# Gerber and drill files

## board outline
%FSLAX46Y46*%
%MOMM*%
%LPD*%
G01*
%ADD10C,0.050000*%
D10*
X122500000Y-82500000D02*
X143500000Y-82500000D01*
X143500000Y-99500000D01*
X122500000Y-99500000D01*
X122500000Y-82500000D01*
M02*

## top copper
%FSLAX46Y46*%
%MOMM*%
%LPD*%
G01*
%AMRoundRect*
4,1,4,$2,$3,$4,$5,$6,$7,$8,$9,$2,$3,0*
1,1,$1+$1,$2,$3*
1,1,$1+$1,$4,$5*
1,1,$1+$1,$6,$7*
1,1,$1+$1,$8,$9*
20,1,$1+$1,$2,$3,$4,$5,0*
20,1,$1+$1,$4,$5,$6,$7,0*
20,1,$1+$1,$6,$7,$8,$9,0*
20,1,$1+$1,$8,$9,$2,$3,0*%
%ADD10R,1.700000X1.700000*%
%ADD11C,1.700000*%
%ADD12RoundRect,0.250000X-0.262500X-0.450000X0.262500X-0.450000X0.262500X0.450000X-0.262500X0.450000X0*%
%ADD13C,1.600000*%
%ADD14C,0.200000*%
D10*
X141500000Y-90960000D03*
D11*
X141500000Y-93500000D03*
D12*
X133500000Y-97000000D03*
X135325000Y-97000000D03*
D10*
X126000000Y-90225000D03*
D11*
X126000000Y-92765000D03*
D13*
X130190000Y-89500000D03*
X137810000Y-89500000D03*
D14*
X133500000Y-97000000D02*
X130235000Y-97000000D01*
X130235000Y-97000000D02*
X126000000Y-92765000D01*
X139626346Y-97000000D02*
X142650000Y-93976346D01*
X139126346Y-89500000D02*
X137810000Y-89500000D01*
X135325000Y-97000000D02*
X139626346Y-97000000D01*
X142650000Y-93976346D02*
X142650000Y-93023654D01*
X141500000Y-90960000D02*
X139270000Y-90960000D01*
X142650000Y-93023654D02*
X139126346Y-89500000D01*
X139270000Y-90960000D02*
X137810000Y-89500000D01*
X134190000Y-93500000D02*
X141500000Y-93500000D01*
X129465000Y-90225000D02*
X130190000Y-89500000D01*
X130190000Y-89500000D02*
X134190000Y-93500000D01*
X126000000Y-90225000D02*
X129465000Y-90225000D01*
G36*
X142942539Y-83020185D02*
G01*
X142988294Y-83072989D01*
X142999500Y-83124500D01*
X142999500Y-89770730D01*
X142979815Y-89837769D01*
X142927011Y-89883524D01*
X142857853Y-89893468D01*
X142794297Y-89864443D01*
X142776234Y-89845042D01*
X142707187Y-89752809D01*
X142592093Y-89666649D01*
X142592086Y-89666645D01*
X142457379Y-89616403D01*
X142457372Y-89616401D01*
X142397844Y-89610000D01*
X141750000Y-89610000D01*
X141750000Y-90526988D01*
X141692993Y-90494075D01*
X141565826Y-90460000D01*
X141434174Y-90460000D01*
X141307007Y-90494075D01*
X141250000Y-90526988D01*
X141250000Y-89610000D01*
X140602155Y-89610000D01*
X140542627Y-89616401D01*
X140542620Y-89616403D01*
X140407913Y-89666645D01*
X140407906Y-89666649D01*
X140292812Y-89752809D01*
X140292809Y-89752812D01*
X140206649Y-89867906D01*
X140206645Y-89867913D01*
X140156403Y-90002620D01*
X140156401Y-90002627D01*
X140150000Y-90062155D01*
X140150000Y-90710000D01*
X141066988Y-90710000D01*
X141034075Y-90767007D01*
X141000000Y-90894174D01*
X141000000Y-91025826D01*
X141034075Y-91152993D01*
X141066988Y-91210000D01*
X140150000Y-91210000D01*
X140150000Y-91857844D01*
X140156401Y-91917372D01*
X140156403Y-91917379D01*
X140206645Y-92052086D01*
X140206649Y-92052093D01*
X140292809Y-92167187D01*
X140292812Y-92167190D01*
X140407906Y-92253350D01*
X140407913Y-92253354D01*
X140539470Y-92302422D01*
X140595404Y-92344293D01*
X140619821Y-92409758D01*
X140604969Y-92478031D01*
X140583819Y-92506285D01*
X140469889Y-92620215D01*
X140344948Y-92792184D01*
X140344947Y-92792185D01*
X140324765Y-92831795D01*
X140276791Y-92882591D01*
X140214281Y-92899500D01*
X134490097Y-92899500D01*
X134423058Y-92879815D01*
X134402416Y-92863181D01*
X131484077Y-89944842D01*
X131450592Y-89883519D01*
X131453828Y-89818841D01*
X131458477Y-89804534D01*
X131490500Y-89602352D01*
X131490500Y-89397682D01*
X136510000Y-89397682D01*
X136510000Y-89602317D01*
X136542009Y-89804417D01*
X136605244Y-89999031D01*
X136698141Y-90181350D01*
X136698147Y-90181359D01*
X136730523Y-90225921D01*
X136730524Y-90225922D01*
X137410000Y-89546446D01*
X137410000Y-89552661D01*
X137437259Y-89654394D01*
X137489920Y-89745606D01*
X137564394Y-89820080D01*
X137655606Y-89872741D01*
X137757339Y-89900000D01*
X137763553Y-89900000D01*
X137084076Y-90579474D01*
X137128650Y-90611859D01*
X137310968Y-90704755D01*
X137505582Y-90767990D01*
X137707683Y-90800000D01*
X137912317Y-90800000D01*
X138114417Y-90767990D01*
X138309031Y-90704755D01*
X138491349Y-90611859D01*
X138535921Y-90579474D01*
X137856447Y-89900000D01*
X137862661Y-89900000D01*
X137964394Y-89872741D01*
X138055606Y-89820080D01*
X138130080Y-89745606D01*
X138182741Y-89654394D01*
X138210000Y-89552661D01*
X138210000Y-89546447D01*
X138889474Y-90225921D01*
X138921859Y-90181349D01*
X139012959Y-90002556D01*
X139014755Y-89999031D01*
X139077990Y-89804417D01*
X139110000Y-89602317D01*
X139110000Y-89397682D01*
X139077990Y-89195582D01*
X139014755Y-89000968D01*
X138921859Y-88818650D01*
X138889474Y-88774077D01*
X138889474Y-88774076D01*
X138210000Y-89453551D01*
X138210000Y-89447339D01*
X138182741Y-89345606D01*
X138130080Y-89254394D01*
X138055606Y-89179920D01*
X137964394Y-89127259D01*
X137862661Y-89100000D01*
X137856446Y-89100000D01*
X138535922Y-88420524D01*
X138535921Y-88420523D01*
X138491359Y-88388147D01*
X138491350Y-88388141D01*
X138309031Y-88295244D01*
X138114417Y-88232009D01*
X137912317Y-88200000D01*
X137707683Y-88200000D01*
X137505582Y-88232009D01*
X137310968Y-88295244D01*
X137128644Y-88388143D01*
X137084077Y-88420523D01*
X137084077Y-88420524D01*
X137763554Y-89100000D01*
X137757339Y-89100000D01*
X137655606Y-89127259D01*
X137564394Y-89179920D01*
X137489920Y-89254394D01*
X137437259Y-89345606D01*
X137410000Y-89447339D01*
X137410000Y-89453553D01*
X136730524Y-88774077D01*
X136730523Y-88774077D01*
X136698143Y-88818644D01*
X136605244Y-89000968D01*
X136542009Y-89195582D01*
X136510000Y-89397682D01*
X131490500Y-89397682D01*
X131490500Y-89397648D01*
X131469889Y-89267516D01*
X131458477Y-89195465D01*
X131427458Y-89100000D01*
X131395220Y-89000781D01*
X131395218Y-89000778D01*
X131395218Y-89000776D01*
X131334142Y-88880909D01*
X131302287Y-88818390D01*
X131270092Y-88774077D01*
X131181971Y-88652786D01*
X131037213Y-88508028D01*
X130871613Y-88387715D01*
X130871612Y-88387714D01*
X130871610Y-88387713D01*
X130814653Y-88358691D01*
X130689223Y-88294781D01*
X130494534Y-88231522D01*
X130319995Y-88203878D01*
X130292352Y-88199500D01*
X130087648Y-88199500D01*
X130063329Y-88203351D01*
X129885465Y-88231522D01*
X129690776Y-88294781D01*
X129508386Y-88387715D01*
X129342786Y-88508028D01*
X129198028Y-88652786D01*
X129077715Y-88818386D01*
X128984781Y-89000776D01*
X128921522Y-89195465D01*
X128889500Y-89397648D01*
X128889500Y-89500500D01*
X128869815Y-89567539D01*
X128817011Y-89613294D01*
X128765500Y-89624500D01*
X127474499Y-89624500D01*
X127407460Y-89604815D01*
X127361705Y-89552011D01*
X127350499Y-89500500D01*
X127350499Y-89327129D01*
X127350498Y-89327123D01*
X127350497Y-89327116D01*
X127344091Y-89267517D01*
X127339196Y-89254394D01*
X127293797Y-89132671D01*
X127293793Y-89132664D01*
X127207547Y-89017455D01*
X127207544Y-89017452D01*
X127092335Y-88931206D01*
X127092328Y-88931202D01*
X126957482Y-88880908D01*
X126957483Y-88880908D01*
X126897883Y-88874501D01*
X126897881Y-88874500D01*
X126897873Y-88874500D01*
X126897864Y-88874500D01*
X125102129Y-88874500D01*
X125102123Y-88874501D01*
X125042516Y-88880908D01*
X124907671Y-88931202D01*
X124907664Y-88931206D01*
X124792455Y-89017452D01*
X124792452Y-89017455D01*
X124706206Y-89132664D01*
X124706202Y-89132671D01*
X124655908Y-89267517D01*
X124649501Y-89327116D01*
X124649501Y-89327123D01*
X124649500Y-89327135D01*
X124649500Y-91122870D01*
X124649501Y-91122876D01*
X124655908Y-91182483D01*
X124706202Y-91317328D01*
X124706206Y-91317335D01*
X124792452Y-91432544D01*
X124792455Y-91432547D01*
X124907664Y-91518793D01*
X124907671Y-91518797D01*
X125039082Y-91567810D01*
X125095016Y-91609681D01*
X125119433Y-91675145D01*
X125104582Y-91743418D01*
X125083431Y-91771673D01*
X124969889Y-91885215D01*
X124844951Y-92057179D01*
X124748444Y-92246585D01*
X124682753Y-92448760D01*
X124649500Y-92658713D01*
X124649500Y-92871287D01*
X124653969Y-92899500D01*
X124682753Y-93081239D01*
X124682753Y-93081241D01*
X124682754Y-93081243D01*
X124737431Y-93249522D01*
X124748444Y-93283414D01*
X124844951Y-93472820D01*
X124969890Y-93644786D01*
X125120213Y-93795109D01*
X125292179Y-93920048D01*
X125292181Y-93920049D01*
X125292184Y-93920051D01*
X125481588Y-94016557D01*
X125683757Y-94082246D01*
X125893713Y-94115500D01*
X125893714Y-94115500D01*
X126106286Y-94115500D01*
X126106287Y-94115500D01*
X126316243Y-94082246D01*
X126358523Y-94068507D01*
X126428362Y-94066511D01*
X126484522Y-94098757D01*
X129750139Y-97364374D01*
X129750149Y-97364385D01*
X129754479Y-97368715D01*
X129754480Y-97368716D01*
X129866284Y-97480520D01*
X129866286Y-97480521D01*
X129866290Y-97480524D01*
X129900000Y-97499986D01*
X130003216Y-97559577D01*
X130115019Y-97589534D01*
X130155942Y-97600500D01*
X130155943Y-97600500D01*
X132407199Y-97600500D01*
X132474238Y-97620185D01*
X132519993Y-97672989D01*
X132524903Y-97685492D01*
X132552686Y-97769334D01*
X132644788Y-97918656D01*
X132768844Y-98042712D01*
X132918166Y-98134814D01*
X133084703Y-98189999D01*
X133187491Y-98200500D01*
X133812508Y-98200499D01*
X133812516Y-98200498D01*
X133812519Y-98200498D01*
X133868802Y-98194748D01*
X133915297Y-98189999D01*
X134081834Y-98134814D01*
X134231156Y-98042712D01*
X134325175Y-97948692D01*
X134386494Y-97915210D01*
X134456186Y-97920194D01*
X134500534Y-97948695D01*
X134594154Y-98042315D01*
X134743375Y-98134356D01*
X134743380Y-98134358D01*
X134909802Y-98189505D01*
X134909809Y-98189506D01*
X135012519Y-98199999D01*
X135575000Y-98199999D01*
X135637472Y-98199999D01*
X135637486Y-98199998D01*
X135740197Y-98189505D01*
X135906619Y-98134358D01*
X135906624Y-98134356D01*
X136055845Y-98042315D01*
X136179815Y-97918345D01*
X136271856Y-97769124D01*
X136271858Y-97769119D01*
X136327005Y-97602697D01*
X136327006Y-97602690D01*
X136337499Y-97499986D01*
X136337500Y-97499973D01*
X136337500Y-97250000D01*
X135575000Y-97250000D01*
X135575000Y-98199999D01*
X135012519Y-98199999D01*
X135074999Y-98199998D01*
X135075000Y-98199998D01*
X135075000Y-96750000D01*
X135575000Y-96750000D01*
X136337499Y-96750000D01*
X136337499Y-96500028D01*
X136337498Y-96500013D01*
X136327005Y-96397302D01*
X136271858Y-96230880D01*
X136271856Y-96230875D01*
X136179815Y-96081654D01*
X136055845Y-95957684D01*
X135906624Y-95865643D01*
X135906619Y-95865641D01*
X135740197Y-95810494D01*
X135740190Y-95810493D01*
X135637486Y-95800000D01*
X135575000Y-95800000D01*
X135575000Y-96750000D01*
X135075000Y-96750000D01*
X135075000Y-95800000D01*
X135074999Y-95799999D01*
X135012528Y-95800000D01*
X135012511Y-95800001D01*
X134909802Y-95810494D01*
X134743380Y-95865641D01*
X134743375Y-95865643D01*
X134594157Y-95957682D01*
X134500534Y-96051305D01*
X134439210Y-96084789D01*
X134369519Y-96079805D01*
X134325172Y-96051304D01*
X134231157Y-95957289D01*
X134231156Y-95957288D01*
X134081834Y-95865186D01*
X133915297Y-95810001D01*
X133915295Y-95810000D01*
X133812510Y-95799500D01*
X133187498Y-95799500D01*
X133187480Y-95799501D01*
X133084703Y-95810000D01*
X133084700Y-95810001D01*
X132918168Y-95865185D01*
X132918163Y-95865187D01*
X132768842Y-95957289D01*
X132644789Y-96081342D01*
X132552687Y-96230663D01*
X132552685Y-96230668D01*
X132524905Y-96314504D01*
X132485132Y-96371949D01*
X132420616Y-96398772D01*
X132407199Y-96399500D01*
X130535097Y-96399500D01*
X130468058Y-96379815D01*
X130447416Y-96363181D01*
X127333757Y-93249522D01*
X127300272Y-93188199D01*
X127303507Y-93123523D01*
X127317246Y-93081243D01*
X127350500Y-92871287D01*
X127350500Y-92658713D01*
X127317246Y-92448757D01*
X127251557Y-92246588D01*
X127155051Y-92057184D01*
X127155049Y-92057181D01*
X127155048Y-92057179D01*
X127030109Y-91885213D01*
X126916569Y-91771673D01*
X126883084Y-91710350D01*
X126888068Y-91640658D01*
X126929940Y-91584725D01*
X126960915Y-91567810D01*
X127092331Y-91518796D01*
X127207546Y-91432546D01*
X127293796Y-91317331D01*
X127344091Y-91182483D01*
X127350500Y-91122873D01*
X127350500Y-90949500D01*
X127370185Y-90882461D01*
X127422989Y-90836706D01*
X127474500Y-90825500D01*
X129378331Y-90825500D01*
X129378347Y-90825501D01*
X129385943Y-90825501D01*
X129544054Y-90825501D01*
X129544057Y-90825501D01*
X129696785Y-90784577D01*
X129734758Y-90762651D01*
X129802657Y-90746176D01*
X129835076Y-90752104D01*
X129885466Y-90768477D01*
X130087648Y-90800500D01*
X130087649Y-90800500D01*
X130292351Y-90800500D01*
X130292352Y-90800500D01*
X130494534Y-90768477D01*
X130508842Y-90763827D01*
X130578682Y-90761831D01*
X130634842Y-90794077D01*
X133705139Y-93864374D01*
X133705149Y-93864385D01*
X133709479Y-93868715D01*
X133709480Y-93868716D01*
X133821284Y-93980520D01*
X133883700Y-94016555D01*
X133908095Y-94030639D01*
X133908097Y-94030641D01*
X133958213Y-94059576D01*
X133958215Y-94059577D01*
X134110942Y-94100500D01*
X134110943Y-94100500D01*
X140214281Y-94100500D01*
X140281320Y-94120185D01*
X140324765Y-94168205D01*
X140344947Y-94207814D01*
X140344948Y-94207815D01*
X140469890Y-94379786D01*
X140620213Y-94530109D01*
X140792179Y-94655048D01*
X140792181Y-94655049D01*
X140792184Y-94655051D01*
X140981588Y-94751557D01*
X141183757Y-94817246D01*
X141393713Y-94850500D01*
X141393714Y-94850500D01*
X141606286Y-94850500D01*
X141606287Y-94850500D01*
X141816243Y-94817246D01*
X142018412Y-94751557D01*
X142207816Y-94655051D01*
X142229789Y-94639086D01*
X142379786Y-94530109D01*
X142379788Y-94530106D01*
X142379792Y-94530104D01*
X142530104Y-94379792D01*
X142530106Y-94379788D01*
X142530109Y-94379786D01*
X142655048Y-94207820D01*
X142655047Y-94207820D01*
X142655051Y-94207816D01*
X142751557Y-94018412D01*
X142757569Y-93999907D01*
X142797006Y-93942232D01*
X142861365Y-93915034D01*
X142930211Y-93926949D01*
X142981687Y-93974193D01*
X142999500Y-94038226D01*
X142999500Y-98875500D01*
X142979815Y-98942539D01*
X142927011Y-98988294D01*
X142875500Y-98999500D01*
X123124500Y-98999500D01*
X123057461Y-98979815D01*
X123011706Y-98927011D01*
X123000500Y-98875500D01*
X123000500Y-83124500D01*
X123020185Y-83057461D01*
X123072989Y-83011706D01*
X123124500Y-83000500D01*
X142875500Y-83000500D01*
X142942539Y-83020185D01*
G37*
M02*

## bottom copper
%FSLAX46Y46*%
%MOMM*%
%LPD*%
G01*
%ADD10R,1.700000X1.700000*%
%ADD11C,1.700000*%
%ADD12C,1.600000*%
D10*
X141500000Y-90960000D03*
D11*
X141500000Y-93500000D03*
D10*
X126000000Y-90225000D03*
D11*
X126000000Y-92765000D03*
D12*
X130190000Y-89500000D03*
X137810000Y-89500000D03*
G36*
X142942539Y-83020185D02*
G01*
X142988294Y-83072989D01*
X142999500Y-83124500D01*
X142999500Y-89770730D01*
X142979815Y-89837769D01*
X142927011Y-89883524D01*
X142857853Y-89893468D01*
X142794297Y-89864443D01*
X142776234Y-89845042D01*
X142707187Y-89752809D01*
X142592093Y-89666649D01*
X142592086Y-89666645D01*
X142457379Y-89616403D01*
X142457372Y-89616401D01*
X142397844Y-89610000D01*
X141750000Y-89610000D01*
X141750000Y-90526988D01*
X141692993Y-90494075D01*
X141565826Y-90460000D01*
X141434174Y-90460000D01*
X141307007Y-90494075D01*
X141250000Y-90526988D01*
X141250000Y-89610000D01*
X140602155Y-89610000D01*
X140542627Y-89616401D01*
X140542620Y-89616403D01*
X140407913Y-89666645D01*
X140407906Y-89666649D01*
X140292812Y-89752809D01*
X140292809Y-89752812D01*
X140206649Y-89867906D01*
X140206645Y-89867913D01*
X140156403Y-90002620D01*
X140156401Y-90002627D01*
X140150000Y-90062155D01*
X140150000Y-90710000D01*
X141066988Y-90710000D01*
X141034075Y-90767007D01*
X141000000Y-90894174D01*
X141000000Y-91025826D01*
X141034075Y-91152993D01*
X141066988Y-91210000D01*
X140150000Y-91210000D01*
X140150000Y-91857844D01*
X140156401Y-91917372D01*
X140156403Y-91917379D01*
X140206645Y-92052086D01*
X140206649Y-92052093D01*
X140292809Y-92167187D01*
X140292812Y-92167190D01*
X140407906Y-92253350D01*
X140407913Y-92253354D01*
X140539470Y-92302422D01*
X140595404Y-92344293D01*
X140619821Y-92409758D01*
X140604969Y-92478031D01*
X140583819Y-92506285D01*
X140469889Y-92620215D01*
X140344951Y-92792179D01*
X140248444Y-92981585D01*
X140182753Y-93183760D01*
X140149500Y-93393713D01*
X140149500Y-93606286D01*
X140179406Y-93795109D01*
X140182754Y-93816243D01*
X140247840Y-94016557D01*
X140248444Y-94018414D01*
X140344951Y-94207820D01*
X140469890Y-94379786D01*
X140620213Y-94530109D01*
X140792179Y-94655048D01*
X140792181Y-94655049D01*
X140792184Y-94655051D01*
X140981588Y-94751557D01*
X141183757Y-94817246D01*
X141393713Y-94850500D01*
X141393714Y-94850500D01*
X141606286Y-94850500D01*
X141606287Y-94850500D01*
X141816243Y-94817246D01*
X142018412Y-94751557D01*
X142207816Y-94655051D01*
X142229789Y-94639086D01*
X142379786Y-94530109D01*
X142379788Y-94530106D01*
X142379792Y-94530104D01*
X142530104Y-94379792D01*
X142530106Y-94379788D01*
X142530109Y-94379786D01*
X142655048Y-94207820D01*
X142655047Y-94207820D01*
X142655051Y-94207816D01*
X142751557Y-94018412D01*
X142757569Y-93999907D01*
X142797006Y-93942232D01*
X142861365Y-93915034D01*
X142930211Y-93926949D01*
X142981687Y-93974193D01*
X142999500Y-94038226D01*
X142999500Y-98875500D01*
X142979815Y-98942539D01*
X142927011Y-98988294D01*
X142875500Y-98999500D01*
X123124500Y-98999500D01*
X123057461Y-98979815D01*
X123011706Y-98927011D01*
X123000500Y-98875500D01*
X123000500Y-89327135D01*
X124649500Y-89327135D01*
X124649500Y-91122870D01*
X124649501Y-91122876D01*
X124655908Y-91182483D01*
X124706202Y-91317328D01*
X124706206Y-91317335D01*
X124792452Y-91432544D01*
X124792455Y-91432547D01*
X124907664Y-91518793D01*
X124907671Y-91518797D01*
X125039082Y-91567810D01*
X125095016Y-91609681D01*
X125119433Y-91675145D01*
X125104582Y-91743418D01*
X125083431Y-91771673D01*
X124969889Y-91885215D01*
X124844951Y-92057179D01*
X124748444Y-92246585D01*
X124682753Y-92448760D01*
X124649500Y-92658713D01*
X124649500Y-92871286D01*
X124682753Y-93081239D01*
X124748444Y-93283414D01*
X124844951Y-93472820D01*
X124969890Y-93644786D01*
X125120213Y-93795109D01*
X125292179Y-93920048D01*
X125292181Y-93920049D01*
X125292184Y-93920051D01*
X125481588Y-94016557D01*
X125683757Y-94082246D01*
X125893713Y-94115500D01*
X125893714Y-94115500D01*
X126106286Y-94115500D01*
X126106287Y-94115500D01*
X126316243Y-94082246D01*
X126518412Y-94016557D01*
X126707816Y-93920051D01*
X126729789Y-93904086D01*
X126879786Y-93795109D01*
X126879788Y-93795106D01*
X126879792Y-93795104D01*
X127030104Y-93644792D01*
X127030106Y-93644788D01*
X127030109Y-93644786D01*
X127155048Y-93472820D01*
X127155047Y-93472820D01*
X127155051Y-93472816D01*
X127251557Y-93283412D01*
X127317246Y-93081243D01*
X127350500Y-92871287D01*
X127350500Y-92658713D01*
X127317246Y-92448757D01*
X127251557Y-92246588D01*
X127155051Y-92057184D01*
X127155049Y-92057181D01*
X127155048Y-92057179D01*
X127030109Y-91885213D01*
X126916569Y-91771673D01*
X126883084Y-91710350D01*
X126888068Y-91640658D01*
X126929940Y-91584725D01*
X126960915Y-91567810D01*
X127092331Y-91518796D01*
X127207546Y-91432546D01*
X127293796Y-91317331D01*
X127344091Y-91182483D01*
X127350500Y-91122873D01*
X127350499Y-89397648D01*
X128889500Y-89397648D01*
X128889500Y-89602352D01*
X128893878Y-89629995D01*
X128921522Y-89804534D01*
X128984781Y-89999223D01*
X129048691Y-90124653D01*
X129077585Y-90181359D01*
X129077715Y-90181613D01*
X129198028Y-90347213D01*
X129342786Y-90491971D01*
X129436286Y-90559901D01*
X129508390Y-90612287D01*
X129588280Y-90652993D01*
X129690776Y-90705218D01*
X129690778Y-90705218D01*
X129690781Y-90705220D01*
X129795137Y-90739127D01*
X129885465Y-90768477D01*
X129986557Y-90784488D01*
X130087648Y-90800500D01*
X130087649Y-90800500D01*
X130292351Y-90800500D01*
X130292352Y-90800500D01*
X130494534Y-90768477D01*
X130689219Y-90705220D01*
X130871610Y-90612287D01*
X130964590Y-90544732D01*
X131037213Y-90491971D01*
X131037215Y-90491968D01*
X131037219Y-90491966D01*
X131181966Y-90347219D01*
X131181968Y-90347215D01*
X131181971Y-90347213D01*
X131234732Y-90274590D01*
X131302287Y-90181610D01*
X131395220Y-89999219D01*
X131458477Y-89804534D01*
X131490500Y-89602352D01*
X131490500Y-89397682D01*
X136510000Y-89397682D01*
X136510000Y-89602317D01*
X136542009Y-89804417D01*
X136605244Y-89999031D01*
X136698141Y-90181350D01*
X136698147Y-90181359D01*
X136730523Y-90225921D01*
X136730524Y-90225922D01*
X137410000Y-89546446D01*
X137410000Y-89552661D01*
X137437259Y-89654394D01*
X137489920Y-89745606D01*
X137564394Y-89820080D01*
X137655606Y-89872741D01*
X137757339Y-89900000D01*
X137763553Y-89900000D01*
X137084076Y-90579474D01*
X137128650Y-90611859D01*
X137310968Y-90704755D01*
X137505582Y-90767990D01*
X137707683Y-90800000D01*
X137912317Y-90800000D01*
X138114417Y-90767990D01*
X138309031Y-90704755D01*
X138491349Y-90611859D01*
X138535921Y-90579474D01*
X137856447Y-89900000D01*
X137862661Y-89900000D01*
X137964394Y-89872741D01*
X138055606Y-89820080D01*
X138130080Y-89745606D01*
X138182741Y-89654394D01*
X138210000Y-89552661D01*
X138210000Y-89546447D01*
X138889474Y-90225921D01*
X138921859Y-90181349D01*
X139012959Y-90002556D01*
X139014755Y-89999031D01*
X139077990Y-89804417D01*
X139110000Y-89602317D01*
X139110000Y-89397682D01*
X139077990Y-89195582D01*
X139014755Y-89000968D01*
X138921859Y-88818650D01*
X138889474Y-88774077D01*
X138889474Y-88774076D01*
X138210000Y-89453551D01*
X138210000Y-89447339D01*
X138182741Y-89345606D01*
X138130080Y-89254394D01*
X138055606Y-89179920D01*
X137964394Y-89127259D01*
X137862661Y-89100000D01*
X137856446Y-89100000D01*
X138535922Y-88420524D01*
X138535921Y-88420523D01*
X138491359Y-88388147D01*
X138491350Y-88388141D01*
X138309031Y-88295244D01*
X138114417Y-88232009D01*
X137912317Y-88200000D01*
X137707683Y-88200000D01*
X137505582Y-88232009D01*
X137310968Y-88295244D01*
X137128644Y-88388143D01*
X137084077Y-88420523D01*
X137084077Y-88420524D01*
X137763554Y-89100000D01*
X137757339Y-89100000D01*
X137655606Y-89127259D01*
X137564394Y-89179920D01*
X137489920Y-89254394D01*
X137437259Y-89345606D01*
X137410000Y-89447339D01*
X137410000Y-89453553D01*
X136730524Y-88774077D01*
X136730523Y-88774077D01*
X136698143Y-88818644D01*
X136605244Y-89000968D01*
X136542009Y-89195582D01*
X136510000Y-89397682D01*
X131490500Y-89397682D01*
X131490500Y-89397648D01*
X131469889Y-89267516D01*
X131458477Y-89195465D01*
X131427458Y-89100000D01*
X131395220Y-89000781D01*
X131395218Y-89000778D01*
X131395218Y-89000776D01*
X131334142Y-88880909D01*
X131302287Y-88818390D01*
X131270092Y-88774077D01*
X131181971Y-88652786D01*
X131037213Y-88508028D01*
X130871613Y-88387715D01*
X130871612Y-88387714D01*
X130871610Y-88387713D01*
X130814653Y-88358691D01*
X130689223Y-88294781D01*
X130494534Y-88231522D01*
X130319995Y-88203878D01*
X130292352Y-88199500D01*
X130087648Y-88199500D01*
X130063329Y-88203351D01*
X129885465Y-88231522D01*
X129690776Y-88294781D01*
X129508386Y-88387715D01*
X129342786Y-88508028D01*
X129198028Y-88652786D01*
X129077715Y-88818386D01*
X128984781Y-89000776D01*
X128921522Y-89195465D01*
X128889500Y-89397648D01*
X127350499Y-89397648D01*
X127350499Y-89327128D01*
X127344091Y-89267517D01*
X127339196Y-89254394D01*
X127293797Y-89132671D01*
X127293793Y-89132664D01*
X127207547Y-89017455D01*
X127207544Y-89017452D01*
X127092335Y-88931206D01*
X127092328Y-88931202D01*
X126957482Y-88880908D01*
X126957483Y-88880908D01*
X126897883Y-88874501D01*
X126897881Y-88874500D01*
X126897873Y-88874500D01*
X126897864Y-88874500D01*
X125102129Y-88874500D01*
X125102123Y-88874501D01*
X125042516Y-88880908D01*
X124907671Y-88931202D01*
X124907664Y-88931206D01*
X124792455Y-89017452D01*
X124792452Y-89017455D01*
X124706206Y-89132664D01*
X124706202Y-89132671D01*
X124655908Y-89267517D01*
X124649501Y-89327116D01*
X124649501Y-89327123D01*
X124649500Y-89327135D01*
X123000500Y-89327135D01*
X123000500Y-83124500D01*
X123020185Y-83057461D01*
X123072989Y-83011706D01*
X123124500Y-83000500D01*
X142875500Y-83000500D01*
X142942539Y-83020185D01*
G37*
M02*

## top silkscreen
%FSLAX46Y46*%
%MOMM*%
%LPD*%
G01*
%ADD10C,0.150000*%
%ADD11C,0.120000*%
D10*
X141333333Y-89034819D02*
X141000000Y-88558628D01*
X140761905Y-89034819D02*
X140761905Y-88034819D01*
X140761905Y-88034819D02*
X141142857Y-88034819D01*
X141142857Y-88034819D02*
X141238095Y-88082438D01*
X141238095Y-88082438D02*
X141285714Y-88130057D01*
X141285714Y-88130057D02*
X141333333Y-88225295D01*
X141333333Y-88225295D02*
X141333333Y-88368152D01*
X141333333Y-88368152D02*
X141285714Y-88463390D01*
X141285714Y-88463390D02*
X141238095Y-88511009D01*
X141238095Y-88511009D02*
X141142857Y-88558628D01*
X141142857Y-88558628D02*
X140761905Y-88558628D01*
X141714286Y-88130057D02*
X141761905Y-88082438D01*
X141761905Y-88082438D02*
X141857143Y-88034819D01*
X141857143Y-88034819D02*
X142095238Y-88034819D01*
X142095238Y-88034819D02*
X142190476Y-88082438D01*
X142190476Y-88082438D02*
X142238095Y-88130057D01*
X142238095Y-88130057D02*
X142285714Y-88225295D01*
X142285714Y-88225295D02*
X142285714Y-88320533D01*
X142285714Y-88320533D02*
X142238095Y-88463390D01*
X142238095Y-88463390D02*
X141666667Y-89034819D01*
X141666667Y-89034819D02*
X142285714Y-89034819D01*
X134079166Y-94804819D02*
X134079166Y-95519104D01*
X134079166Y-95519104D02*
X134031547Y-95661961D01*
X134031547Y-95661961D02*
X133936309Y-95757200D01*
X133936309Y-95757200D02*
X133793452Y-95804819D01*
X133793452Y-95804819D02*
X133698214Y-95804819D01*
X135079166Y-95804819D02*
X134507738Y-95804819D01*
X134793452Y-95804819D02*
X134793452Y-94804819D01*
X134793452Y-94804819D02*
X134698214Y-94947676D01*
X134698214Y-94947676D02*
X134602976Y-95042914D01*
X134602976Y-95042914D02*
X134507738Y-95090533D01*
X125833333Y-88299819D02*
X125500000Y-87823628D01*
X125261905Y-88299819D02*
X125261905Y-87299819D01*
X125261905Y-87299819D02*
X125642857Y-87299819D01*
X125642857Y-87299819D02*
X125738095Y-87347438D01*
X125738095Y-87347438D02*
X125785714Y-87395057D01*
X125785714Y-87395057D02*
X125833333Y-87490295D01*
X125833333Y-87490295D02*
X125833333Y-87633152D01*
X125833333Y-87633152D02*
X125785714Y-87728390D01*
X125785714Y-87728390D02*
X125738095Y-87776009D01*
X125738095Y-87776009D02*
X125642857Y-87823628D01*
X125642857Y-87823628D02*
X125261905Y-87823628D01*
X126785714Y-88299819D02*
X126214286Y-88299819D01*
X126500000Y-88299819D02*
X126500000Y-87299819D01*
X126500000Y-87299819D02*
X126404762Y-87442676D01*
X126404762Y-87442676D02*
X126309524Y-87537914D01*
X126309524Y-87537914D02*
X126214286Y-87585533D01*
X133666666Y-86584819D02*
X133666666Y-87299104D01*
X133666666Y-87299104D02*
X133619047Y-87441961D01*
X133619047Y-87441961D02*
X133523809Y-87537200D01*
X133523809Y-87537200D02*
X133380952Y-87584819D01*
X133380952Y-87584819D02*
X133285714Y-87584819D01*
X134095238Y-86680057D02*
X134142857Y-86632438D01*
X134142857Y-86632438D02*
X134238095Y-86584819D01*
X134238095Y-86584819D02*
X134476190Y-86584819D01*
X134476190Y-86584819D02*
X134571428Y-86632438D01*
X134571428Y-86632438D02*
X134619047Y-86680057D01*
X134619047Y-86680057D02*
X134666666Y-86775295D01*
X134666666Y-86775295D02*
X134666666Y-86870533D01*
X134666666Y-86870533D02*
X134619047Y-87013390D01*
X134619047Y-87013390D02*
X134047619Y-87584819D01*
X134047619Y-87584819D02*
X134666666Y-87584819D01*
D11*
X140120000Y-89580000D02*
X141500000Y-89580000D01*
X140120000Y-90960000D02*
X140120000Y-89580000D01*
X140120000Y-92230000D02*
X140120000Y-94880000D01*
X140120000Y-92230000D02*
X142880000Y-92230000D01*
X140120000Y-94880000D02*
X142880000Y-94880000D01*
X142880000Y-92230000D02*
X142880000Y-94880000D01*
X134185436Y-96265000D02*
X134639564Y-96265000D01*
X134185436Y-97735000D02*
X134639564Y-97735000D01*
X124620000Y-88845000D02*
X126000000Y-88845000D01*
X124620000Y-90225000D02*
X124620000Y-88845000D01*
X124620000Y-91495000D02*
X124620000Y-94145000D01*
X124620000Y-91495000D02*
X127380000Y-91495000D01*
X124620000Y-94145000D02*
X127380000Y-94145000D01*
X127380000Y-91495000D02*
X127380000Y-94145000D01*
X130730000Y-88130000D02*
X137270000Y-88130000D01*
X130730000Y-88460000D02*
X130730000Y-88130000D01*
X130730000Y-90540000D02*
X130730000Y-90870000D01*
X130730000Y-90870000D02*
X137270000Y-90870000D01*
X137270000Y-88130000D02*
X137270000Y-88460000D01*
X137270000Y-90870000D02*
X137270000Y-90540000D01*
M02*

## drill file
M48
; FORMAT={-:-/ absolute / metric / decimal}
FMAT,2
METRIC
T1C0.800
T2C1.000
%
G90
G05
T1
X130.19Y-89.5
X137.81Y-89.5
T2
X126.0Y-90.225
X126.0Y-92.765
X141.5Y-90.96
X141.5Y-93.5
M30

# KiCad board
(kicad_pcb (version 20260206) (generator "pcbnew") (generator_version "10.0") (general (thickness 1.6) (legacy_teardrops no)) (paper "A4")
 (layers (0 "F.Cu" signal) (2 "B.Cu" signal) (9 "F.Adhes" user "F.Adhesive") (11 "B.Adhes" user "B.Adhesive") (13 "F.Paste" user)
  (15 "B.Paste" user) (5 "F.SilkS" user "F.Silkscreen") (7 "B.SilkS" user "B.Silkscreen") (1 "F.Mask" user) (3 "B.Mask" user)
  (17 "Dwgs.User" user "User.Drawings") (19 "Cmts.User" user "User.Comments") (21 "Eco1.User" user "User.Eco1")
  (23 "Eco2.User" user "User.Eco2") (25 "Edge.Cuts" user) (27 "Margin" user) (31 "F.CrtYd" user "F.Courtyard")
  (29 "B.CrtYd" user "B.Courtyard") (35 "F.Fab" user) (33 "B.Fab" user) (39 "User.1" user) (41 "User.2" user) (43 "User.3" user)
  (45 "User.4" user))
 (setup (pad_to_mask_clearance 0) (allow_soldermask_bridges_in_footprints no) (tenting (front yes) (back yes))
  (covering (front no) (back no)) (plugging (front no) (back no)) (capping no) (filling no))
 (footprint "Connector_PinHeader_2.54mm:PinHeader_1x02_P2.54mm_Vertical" (layer "F.Cu") (at 141.5 90.96)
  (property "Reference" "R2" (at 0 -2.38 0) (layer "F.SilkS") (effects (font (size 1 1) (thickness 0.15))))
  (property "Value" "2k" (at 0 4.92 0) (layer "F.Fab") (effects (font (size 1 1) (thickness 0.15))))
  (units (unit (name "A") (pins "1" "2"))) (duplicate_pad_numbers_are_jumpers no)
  (fp_line (start -1.38 -1.38) (end 0 -1.38) (stroke (width 0.12) (type solid)) (layer "F.SilkS"))
  (fp_line (start -1.38 0) (end -1.38 -1.38) (stroke (width 0.12) (type solid)) (layer "F.SilkS"))
  (fp_line (start -1.38 1.27) (end -1.38 3.92) (stroke (width 0.12) (type solid)) (layer "F.SilkS"))
  (fp_line (start -1.38 1.27) (end 1.38 1.27) (stroke (width 0.12) (type solid)) (layer "F.SilkS"))
  (fp_line (start -1.38 3.92) (end 1.38 3.92) (stroke (width 0.12) (type solid)) (layer "F.SilkS"))
  (fp_line (start 1.38 1.27) (end 1.38 3.92) (stroke (width 0.12) (type solid)) (layer "F.SilkS"))
  (pad "1" thru_hole rect (at 0 0) (size 1.7 1.7) (drill 1) (layers "*.Cu" "*.Mask") (remove_unused_layers no) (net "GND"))
  (pad "2" thru_hole circle (at 0 2.54) (size 1.7 1.7) (drill 1) (layers "*.Cu" "*.Mask") (remove_unused_layers no) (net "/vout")))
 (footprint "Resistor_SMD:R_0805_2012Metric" (layer "F.Cu") (at 134.4125 97)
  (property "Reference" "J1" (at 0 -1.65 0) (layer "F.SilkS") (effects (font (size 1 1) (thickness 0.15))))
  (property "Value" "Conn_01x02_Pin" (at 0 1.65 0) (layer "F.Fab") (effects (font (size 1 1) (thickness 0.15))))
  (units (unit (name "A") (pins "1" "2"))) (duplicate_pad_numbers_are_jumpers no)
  (fp_line (start -0.227064 -0.735) (end 0.227064 -0.735) (stroke (width 0.12) (type solid)) (layer "F.SilkS"))
  (fp_line (start -0.227064 0.735) (end 0.227064 0.735) (stroke (width 0.12) (type solid)) (layer "F.SilkS"))
  (pad "1" smd roundrect (at -0.9125 0) (size 1.025 1.4) (layers "F.Cu" "F.Mask" "F.Paste") (roundrect_rratio 0.243902)
   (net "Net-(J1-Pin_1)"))
  (pad "2" smd roundrect (at 0.9125 0) (size 1.025 1.4) (layers "F.Cu" "F.Mask" "F.Paste") (roundrect_rratio 0.243902) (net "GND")))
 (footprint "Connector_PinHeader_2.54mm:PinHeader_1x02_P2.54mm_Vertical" (layer "F.Cu") (at 126 90.225)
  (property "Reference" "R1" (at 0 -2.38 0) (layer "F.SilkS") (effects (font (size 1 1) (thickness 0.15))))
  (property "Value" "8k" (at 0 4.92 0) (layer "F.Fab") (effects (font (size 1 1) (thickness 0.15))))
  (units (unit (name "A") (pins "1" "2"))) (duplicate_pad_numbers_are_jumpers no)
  (fp_line (start -1.38 -1.38) (end 0 -1.38) (stroke (width 0.12) (type solid)) (layer "F.SilkS"))
  (fp_line (start -1.38 0) (end -1.38 -1.38) (stroke (width 0.12) (type solid)) (layer "F.SilkS"))
  (fp_line (start -1.38 1.27) (end -1.38 3.92) (stroke (width 0.12) (type solid)) (layer "F.SilkS"))
  (fp_line (start -1.38 1.27) (end 1.38 1.27) (stroke (width 0.12) (type solid)) (layer "F.SilkS"))
  (fp_line (start -1.38 3.92) (end 1.38 3.92) (stroke (width 0.12) (type solid)) (layer "F.SilkS"))
  (fp_line (start 1.38 1.27) (end 1.38 3.92) (stroke (width 0.12) (type solid)) (layer "F.SilkS"))
  (pad "1" thru_hole rect (at 0 0) (size 1.7 1.7) (drill 1) (layers "*.Cu" "*.Mask") (remove_unused_layers no) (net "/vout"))
  (pad "2" thru_hole circle (at 0 2.54) (size 1.7 1.7) (drill 1) (layers "*.Cu" "*.Mask") (remove_unused_layers no) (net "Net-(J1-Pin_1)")))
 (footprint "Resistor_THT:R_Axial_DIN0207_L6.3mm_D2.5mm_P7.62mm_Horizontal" (layer "F.Cu") (at 130.19 89.5)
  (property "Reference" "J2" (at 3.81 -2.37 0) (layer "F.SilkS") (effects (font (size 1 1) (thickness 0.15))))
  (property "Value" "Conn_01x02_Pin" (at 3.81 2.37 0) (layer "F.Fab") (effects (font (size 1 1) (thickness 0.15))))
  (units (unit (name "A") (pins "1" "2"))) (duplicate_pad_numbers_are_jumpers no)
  (fp_line (start 0.54 -1.37) (end 7.08 -1.37) (stroke (width 0.12) (type solid)) (layer "F.SilkS"))
  (fp_line (start 0.54 -1.04) (end 0.54 -1.37) (stroke (width 0.12) (type solid)) (layer "F.SilkS"))
  (fp_line (start 0.54 1.04) (end 0.54 1.37) (stroke (width 0.12) (type solid)) (layer "F.SilkS"))
  (fp_line (start 0.54 1.37) (end 7.08 1.37) (stroke (width 0.12) (type solid)) (layer "F.SilkS"))
  (fp_line (start 7.08 -1.37) (end 7.08 -1.04) (stroke (width 0.12) (type solid)) (layer "F.SilkS"))
  (fp_line (start 7.08 1.37) (end 7.08 1.04) (stroke (width 0.12) (type solid)) (layer "F.SilkS"))
  (pad "1" thru_hole circle (at 0 0) (size 1.6 1.6) (drill 0.8) (layers "*.Cu" "*.Mask") (remove_unused_layers no) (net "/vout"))
  (pad "2" thru_hole circle (at 7.62 0) (size 1.6 1.6) (drill 0.8) (layers "*.Cu" "*.Mask") (remove_unused_layers no) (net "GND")))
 (gr_rect (start 122.5 82.5) (end 143.5 99.5) (stroke (width 0.05) (type default)) (fill no) (layer "Edge.Cuts"))
 (segment (start 133.5 97) (end 130.235 97) (width 0.2) (layer "F.Cu") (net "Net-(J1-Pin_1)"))
 (segment (start 130.235 97) (end 126 92.765) (width 0.2) (layer "F.Cu") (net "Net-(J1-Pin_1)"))
 (segment (start 139.626346 97) (end 142.65 93.976346) (width 0.2) (layer "F.Cu") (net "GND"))
 (segment (start 139.126346 89.5) (end 137.81 89.5) (width 0.2) (layer "F.Cu") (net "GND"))
 (segment (start 135.325 97) (end 139.626346 97) (width 0.2) (layer "F.Cu") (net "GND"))
 (segment (start 142.65 93.976346) (end 142.65 93.023654) (width 0.2) (layer "F.Cu") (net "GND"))
 (segment (start 141.5 90.96) (end 139.27 90.96) (width 0.2) (layer "F.Cu") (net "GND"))
 (segment (start 142.65 93.023654) (end 139.126346 89.5) (width 0.2) (layer "F.Cu") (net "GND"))
 (segment (start 139.27 90.96) (end 137.81 89.5) (width 0.2) (layer "F.Cu") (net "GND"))
 (segment (start 134.19 93.5) (end 141.5 93.5) (width 0.2) (layer "F.Cu") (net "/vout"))
 (segment (start 129.465 90.225) (end 130.19 89.5) (width 0.2) (layer "F.Cu") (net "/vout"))
 (segment (start 130.19 89.5) (end 134.19 93.5) (width 0.2) (layer "F.Cu") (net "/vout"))
 (segment (start 126 90.225) (end 129.465 90.225) (width 0.2) (layer "F.Cu") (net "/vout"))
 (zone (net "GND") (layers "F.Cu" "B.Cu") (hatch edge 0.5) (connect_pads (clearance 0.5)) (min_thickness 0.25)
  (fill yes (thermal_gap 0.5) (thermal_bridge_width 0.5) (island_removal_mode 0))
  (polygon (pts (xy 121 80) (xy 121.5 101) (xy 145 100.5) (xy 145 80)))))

